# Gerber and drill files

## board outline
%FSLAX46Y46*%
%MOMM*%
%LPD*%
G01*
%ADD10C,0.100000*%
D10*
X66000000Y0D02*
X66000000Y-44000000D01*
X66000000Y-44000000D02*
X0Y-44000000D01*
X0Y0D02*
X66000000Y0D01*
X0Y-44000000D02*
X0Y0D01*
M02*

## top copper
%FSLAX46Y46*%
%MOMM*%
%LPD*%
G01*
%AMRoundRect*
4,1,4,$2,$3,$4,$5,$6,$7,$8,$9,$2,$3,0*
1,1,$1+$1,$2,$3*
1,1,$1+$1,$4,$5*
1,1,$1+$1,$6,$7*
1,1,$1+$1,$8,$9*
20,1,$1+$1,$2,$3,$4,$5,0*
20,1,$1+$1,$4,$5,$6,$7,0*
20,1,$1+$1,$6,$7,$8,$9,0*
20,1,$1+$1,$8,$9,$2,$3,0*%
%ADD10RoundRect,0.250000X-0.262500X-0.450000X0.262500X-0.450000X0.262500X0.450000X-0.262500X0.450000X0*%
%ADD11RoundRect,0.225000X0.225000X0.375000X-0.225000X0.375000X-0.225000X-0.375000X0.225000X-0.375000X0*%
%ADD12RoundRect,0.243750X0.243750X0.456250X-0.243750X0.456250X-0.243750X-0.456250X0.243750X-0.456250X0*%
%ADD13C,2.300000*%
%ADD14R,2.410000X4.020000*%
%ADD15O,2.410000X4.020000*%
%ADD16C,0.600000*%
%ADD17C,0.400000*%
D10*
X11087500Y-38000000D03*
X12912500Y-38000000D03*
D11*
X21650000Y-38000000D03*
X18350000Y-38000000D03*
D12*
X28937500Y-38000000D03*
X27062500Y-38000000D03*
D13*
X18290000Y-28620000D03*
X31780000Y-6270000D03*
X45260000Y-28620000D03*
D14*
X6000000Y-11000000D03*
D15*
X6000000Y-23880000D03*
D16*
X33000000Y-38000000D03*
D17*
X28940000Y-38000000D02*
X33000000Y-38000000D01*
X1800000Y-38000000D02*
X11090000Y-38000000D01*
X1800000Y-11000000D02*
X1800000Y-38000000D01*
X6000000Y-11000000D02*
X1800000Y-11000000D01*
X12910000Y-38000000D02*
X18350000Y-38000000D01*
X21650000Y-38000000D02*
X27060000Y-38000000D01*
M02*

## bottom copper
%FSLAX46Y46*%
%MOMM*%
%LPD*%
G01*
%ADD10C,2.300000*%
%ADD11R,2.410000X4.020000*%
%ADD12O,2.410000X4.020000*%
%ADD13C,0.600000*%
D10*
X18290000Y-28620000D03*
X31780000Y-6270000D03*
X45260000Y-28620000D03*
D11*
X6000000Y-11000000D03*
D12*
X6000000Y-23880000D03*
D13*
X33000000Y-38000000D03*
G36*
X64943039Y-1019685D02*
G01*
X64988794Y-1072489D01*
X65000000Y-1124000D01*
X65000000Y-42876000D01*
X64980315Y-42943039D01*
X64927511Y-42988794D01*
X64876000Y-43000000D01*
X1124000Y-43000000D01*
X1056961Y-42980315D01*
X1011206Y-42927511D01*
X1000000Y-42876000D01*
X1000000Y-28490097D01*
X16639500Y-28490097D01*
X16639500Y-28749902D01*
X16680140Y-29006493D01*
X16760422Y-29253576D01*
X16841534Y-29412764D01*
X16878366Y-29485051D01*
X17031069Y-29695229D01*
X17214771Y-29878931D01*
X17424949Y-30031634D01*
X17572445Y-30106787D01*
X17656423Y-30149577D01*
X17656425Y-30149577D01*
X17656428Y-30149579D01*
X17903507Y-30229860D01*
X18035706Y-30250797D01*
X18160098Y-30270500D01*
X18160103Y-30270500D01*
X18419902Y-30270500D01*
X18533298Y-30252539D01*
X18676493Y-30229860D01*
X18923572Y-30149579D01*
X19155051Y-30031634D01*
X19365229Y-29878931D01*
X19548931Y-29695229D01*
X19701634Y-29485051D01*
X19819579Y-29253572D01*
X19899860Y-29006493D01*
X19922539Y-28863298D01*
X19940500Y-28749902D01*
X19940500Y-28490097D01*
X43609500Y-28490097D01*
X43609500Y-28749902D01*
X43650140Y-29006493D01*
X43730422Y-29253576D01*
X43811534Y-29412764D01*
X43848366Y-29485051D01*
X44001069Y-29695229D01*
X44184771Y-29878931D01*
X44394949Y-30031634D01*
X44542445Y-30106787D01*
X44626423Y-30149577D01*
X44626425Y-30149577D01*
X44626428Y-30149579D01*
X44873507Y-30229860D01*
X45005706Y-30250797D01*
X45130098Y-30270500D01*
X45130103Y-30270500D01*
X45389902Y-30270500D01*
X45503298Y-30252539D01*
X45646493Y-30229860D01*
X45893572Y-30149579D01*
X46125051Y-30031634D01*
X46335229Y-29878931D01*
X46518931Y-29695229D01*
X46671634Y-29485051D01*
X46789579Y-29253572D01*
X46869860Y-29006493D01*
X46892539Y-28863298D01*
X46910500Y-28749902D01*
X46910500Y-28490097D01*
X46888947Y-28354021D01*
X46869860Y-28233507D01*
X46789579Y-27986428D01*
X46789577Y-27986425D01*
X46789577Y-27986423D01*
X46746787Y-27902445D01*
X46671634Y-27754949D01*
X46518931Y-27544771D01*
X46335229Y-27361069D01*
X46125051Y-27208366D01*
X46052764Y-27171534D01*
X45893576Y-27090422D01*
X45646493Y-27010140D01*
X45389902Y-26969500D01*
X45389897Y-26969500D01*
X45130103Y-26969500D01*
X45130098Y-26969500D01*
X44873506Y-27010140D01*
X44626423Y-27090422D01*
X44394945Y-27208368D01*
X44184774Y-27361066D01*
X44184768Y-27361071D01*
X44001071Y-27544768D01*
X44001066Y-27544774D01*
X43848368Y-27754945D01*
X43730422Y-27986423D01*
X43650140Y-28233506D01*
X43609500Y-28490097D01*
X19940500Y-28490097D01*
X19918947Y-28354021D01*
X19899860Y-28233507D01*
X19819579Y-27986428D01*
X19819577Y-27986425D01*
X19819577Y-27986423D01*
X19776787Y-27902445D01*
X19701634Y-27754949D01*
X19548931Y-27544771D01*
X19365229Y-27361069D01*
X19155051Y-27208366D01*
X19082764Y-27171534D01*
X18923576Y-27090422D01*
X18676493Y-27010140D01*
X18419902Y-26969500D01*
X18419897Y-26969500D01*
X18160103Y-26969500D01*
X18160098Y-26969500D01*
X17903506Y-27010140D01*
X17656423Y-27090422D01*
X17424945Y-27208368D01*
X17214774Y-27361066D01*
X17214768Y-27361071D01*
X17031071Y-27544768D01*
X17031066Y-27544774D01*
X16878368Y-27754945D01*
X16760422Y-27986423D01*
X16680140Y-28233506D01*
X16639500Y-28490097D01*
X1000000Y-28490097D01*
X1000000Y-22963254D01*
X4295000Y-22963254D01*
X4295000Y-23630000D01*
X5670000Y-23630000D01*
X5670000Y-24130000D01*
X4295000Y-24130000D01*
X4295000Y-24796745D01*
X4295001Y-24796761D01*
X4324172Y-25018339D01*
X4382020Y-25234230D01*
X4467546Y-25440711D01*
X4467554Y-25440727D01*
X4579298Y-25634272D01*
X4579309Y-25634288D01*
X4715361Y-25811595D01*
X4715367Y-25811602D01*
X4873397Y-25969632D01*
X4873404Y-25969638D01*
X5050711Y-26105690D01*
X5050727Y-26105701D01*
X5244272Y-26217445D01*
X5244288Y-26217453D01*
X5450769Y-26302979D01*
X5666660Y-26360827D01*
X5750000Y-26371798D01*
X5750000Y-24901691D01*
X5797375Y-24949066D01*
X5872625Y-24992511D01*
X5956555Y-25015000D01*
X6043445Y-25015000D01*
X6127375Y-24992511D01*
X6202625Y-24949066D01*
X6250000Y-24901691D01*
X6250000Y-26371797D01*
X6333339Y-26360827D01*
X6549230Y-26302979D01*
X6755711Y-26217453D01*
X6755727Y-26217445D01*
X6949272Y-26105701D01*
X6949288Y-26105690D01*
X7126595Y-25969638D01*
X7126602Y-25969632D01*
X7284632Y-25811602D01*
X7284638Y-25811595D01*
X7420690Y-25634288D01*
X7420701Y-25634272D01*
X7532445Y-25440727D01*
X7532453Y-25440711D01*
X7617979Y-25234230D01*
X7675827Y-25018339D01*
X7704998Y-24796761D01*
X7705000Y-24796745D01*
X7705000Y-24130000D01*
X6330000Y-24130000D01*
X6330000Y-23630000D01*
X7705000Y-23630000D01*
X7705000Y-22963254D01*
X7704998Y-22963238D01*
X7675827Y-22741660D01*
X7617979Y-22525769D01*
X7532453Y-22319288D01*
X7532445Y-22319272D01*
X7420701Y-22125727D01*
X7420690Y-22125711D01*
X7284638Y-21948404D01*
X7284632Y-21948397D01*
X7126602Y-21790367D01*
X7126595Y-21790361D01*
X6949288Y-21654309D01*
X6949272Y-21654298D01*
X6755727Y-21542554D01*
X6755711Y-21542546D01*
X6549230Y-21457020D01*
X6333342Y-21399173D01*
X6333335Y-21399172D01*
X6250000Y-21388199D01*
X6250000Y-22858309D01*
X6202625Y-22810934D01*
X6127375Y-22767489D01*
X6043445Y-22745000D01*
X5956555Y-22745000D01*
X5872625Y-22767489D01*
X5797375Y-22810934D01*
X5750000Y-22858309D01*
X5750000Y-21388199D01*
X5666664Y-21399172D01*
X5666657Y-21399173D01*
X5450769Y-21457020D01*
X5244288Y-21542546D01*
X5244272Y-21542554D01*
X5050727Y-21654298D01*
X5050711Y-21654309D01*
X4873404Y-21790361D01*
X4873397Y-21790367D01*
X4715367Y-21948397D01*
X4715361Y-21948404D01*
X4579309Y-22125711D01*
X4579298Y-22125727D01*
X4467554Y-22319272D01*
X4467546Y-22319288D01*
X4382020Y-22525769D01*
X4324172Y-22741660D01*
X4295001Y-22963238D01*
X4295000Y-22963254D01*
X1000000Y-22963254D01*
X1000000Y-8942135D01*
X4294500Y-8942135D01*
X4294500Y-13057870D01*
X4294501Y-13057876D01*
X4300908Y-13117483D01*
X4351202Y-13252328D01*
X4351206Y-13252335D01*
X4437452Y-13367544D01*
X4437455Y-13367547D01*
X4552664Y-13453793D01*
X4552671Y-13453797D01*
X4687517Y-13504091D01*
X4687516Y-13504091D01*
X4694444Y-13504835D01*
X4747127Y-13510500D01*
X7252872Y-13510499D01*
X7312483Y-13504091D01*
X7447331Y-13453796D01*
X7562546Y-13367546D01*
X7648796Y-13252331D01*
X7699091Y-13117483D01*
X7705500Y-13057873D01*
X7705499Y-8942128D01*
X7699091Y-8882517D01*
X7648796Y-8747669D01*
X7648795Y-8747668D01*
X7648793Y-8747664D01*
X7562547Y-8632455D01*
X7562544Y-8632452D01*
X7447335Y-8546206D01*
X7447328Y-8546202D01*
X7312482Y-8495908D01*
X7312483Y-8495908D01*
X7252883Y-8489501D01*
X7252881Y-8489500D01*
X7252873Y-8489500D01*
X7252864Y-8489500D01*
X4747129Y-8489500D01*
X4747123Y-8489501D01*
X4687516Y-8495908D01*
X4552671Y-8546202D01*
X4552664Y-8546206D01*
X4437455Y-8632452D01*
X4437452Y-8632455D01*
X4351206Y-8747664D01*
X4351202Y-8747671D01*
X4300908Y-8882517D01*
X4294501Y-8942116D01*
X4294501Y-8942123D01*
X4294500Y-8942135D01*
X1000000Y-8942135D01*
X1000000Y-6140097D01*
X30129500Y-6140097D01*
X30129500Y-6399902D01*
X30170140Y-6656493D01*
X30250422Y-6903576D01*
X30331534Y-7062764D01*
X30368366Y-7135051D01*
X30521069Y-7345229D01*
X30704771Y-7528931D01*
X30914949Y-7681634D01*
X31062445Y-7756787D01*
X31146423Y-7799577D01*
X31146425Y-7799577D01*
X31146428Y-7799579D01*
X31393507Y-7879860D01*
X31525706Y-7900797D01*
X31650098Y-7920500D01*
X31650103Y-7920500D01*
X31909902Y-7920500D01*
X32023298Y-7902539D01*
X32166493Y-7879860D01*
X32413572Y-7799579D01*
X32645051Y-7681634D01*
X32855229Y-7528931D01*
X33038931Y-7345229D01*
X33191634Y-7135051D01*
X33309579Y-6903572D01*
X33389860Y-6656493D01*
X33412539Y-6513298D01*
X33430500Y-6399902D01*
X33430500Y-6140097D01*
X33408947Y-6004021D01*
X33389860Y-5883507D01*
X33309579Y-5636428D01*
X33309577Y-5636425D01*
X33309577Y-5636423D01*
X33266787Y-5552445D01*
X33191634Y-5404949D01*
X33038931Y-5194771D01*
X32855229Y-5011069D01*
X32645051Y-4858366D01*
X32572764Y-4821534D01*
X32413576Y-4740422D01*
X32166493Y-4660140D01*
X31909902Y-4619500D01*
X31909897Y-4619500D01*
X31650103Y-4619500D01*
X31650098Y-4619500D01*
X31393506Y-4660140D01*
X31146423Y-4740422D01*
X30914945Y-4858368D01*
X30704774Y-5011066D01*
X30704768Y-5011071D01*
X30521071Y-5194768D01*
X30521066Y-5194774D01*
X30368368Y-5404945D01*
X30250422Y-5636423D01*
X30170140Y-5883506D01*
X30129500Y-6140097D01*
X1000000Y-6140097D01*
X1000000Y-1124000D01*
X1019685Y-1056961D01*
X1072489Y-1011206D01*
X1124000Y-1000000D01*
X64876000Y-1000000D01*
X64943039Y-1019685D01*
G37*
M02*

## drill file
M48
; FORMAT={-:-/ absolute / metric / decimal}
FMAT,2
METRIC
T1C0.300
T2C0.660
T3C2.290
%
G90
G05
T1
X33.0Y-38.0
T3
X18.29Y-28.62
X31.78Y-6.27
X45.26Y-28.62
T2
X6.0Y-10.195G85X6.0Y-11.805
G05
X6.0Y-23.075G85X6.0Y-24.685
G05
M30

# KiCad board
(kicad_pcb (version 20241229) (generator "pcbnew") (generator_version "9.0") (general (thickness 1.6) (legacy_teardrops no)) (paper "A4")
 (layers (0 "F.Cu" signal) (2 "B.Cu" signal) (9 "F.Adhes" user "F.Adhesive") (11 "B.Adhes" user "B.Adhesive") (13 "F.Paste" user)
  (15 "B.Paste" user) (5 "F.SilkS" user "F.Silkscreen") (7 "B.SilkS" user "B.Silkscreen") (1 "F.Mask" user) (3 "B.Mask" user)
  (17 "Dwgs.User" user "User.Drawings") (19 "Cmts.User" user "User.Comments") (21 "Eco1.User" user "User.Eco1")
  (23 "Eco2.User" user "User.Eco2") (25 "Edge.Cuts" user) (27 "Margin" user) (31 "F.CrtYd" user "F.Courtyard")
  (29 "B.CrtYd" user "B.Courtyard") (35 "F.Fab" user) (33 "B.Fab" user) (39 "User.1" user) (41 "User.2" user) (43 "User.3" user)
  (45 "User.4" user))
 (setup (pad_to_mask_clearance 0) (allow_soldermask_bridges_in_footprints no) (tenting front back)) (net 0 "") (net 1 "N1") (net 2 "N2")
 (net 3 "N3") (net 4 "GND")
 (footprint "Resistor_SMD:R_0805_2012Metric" (layer "F.Cu") (at 12 38)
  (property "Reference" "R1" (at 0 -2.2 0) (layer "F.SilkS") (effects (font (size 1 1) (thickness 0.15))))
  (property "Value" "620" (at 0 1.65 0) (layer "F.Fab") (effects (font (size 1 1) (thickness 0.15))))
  (pad "1" smd roundrect (at -0.9125 0) (size 1.025 1.4) (layers "F.Cu" "F.Mask" "F.Paste") (roundrect_rratio 0.243902) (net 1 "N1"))
  (pad "2" smd roundrect (at 0.9125 0) (size 1.025 1.4) (layers "F.Cu" "F.Mask" "F.Paste") (roundrect_rratio 0.243902) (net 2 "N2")))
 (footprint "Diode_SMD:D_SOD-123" (layer "F.Cu") (at 20 38 180)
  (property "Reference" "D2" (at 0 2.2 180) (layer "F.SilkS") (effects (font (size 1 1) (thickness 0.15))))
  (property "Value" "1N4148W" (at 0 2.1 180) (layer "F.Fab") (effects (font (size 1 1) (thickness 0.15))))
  (pad "1" smd roundrect (at -1.65 0 180) (size 0.9 1.2) (layers "F.Cu" "F.Mask" "F.Paste") (roundrect_rratio 0.25) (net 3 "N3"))
  (pad "2" smd roundrect (at 1.65 0 180) (size 0.9 1.2) (layers "F.Cu" "F.Mask" "F.Paste") (roundrect_rratio 0.25) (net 2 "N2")))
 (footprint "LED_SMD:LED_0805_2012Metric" (layer "F.Cu") (at 28 38 180)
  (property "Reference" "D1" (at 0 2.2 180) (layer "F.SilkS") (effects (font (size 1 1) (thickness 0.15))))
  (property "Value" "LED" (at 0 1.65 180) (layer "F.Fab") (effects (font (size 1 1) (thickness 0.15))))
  (pad "1" smd roundrect (at -0.9375 0 180) (size 0.975 1.4) (layers "F.Cu" "F.Mask" "F.Paste") (roundrect_rratio 0.25) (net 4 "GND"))
  (pad "2" smd roundrect (at 0.9375 0 180) (size 0.975 1.4) (layers "F.Cu" "F.Mask" "F.Paste") (roundrect_rratio 0.25) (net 3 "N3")))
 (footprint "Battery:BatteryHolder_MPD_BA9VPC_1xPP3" (layer "F.Cu") (at 6 11)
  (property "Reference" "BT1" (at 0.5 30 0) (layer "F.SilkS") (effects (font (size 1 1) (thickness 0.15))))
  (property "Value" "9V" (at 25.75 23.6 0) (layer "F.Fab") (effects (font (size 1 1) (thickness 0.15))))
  (pad "" np_thru_hole circle (at 12.29 17.62) (size 2.3 2.3) (drill 2.29) (layers "*.Cu" "*.Mask"))
  (pad "" np_thru_hole circle (at 25.78 -4.73) (size 2.3 2.3) (drill 2.29) (layers "*.Cu" "*.Mask"))
  (pad "" np_thru_hole circle (at 39.26 17.62) (size 2.3 2.3) (drill 2.29) (layers "*.Cu" "*.Mask"))
  (pad "1" thru_hole rect (at 0 0) (size 2.41 4.02) (drill oval 0.66 2.27) (layers "*.Cu" "*.Mask") (remove_unused_layers no) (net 1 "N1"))
  (pad "2" thru_hole oval (at 0 12.88) (size 2.41 4.02) (drill oval 0.66 2.27) (layers "*.Cu" "*.Mask") (remove_unused_layers no)
   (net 4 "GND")))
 (gr_line (start 66 0) (end 66 44) (stroke (width 0.1) (type default)) (layer "Edge.Cuts"))
 (gr_line (start 66 44) (end 0 44) (stroke (width 0.1) (type default)) (layer "Edge.Cuts"))
 (gr_line (start 0 0) (end 66 0) (stroke (width 0.1) (type default)) (layer "Edge.Cuts"))
 (gr_line (start 0 44) (end 0 0) (stroke (width 0.1) (type default)) (layer "Edge.Cuts"))
 (segment (start 28.94 38) (end 33 38) (width 0.4) (layer "F.Cu") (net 4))
 (via (at 33 38) (size 0.6) (drill 0.3) (layers "F.Cu" "B.Cu") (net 4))
 (segment (start 1.8 38) (end 11.09 38) (width 0.4) (layer "F.Cu") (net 1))
 (segment (start 1.8 11) (end 1.8 38) (width 0.4) (layer "F.Cu") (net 1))
 (segment (start 6 11) (end 1.8 11) (width 0.4) (layer "F.Cu") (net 1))
 (segment (start 12.91 38) (end 18.35 38) (width 0.4) (layer "F.Cu") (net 2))
 (segment (start 21.65 38) (end 27.06 38) (width 0.4) (layer "F.Cu") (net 3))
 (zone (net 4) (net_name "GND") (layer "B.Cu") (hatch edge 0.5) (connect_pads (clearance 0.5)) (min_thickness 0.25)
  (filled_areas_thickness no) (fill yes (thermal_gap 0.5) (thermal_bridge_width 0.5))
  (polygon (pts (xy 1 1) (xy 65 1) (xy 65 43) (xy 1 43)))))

